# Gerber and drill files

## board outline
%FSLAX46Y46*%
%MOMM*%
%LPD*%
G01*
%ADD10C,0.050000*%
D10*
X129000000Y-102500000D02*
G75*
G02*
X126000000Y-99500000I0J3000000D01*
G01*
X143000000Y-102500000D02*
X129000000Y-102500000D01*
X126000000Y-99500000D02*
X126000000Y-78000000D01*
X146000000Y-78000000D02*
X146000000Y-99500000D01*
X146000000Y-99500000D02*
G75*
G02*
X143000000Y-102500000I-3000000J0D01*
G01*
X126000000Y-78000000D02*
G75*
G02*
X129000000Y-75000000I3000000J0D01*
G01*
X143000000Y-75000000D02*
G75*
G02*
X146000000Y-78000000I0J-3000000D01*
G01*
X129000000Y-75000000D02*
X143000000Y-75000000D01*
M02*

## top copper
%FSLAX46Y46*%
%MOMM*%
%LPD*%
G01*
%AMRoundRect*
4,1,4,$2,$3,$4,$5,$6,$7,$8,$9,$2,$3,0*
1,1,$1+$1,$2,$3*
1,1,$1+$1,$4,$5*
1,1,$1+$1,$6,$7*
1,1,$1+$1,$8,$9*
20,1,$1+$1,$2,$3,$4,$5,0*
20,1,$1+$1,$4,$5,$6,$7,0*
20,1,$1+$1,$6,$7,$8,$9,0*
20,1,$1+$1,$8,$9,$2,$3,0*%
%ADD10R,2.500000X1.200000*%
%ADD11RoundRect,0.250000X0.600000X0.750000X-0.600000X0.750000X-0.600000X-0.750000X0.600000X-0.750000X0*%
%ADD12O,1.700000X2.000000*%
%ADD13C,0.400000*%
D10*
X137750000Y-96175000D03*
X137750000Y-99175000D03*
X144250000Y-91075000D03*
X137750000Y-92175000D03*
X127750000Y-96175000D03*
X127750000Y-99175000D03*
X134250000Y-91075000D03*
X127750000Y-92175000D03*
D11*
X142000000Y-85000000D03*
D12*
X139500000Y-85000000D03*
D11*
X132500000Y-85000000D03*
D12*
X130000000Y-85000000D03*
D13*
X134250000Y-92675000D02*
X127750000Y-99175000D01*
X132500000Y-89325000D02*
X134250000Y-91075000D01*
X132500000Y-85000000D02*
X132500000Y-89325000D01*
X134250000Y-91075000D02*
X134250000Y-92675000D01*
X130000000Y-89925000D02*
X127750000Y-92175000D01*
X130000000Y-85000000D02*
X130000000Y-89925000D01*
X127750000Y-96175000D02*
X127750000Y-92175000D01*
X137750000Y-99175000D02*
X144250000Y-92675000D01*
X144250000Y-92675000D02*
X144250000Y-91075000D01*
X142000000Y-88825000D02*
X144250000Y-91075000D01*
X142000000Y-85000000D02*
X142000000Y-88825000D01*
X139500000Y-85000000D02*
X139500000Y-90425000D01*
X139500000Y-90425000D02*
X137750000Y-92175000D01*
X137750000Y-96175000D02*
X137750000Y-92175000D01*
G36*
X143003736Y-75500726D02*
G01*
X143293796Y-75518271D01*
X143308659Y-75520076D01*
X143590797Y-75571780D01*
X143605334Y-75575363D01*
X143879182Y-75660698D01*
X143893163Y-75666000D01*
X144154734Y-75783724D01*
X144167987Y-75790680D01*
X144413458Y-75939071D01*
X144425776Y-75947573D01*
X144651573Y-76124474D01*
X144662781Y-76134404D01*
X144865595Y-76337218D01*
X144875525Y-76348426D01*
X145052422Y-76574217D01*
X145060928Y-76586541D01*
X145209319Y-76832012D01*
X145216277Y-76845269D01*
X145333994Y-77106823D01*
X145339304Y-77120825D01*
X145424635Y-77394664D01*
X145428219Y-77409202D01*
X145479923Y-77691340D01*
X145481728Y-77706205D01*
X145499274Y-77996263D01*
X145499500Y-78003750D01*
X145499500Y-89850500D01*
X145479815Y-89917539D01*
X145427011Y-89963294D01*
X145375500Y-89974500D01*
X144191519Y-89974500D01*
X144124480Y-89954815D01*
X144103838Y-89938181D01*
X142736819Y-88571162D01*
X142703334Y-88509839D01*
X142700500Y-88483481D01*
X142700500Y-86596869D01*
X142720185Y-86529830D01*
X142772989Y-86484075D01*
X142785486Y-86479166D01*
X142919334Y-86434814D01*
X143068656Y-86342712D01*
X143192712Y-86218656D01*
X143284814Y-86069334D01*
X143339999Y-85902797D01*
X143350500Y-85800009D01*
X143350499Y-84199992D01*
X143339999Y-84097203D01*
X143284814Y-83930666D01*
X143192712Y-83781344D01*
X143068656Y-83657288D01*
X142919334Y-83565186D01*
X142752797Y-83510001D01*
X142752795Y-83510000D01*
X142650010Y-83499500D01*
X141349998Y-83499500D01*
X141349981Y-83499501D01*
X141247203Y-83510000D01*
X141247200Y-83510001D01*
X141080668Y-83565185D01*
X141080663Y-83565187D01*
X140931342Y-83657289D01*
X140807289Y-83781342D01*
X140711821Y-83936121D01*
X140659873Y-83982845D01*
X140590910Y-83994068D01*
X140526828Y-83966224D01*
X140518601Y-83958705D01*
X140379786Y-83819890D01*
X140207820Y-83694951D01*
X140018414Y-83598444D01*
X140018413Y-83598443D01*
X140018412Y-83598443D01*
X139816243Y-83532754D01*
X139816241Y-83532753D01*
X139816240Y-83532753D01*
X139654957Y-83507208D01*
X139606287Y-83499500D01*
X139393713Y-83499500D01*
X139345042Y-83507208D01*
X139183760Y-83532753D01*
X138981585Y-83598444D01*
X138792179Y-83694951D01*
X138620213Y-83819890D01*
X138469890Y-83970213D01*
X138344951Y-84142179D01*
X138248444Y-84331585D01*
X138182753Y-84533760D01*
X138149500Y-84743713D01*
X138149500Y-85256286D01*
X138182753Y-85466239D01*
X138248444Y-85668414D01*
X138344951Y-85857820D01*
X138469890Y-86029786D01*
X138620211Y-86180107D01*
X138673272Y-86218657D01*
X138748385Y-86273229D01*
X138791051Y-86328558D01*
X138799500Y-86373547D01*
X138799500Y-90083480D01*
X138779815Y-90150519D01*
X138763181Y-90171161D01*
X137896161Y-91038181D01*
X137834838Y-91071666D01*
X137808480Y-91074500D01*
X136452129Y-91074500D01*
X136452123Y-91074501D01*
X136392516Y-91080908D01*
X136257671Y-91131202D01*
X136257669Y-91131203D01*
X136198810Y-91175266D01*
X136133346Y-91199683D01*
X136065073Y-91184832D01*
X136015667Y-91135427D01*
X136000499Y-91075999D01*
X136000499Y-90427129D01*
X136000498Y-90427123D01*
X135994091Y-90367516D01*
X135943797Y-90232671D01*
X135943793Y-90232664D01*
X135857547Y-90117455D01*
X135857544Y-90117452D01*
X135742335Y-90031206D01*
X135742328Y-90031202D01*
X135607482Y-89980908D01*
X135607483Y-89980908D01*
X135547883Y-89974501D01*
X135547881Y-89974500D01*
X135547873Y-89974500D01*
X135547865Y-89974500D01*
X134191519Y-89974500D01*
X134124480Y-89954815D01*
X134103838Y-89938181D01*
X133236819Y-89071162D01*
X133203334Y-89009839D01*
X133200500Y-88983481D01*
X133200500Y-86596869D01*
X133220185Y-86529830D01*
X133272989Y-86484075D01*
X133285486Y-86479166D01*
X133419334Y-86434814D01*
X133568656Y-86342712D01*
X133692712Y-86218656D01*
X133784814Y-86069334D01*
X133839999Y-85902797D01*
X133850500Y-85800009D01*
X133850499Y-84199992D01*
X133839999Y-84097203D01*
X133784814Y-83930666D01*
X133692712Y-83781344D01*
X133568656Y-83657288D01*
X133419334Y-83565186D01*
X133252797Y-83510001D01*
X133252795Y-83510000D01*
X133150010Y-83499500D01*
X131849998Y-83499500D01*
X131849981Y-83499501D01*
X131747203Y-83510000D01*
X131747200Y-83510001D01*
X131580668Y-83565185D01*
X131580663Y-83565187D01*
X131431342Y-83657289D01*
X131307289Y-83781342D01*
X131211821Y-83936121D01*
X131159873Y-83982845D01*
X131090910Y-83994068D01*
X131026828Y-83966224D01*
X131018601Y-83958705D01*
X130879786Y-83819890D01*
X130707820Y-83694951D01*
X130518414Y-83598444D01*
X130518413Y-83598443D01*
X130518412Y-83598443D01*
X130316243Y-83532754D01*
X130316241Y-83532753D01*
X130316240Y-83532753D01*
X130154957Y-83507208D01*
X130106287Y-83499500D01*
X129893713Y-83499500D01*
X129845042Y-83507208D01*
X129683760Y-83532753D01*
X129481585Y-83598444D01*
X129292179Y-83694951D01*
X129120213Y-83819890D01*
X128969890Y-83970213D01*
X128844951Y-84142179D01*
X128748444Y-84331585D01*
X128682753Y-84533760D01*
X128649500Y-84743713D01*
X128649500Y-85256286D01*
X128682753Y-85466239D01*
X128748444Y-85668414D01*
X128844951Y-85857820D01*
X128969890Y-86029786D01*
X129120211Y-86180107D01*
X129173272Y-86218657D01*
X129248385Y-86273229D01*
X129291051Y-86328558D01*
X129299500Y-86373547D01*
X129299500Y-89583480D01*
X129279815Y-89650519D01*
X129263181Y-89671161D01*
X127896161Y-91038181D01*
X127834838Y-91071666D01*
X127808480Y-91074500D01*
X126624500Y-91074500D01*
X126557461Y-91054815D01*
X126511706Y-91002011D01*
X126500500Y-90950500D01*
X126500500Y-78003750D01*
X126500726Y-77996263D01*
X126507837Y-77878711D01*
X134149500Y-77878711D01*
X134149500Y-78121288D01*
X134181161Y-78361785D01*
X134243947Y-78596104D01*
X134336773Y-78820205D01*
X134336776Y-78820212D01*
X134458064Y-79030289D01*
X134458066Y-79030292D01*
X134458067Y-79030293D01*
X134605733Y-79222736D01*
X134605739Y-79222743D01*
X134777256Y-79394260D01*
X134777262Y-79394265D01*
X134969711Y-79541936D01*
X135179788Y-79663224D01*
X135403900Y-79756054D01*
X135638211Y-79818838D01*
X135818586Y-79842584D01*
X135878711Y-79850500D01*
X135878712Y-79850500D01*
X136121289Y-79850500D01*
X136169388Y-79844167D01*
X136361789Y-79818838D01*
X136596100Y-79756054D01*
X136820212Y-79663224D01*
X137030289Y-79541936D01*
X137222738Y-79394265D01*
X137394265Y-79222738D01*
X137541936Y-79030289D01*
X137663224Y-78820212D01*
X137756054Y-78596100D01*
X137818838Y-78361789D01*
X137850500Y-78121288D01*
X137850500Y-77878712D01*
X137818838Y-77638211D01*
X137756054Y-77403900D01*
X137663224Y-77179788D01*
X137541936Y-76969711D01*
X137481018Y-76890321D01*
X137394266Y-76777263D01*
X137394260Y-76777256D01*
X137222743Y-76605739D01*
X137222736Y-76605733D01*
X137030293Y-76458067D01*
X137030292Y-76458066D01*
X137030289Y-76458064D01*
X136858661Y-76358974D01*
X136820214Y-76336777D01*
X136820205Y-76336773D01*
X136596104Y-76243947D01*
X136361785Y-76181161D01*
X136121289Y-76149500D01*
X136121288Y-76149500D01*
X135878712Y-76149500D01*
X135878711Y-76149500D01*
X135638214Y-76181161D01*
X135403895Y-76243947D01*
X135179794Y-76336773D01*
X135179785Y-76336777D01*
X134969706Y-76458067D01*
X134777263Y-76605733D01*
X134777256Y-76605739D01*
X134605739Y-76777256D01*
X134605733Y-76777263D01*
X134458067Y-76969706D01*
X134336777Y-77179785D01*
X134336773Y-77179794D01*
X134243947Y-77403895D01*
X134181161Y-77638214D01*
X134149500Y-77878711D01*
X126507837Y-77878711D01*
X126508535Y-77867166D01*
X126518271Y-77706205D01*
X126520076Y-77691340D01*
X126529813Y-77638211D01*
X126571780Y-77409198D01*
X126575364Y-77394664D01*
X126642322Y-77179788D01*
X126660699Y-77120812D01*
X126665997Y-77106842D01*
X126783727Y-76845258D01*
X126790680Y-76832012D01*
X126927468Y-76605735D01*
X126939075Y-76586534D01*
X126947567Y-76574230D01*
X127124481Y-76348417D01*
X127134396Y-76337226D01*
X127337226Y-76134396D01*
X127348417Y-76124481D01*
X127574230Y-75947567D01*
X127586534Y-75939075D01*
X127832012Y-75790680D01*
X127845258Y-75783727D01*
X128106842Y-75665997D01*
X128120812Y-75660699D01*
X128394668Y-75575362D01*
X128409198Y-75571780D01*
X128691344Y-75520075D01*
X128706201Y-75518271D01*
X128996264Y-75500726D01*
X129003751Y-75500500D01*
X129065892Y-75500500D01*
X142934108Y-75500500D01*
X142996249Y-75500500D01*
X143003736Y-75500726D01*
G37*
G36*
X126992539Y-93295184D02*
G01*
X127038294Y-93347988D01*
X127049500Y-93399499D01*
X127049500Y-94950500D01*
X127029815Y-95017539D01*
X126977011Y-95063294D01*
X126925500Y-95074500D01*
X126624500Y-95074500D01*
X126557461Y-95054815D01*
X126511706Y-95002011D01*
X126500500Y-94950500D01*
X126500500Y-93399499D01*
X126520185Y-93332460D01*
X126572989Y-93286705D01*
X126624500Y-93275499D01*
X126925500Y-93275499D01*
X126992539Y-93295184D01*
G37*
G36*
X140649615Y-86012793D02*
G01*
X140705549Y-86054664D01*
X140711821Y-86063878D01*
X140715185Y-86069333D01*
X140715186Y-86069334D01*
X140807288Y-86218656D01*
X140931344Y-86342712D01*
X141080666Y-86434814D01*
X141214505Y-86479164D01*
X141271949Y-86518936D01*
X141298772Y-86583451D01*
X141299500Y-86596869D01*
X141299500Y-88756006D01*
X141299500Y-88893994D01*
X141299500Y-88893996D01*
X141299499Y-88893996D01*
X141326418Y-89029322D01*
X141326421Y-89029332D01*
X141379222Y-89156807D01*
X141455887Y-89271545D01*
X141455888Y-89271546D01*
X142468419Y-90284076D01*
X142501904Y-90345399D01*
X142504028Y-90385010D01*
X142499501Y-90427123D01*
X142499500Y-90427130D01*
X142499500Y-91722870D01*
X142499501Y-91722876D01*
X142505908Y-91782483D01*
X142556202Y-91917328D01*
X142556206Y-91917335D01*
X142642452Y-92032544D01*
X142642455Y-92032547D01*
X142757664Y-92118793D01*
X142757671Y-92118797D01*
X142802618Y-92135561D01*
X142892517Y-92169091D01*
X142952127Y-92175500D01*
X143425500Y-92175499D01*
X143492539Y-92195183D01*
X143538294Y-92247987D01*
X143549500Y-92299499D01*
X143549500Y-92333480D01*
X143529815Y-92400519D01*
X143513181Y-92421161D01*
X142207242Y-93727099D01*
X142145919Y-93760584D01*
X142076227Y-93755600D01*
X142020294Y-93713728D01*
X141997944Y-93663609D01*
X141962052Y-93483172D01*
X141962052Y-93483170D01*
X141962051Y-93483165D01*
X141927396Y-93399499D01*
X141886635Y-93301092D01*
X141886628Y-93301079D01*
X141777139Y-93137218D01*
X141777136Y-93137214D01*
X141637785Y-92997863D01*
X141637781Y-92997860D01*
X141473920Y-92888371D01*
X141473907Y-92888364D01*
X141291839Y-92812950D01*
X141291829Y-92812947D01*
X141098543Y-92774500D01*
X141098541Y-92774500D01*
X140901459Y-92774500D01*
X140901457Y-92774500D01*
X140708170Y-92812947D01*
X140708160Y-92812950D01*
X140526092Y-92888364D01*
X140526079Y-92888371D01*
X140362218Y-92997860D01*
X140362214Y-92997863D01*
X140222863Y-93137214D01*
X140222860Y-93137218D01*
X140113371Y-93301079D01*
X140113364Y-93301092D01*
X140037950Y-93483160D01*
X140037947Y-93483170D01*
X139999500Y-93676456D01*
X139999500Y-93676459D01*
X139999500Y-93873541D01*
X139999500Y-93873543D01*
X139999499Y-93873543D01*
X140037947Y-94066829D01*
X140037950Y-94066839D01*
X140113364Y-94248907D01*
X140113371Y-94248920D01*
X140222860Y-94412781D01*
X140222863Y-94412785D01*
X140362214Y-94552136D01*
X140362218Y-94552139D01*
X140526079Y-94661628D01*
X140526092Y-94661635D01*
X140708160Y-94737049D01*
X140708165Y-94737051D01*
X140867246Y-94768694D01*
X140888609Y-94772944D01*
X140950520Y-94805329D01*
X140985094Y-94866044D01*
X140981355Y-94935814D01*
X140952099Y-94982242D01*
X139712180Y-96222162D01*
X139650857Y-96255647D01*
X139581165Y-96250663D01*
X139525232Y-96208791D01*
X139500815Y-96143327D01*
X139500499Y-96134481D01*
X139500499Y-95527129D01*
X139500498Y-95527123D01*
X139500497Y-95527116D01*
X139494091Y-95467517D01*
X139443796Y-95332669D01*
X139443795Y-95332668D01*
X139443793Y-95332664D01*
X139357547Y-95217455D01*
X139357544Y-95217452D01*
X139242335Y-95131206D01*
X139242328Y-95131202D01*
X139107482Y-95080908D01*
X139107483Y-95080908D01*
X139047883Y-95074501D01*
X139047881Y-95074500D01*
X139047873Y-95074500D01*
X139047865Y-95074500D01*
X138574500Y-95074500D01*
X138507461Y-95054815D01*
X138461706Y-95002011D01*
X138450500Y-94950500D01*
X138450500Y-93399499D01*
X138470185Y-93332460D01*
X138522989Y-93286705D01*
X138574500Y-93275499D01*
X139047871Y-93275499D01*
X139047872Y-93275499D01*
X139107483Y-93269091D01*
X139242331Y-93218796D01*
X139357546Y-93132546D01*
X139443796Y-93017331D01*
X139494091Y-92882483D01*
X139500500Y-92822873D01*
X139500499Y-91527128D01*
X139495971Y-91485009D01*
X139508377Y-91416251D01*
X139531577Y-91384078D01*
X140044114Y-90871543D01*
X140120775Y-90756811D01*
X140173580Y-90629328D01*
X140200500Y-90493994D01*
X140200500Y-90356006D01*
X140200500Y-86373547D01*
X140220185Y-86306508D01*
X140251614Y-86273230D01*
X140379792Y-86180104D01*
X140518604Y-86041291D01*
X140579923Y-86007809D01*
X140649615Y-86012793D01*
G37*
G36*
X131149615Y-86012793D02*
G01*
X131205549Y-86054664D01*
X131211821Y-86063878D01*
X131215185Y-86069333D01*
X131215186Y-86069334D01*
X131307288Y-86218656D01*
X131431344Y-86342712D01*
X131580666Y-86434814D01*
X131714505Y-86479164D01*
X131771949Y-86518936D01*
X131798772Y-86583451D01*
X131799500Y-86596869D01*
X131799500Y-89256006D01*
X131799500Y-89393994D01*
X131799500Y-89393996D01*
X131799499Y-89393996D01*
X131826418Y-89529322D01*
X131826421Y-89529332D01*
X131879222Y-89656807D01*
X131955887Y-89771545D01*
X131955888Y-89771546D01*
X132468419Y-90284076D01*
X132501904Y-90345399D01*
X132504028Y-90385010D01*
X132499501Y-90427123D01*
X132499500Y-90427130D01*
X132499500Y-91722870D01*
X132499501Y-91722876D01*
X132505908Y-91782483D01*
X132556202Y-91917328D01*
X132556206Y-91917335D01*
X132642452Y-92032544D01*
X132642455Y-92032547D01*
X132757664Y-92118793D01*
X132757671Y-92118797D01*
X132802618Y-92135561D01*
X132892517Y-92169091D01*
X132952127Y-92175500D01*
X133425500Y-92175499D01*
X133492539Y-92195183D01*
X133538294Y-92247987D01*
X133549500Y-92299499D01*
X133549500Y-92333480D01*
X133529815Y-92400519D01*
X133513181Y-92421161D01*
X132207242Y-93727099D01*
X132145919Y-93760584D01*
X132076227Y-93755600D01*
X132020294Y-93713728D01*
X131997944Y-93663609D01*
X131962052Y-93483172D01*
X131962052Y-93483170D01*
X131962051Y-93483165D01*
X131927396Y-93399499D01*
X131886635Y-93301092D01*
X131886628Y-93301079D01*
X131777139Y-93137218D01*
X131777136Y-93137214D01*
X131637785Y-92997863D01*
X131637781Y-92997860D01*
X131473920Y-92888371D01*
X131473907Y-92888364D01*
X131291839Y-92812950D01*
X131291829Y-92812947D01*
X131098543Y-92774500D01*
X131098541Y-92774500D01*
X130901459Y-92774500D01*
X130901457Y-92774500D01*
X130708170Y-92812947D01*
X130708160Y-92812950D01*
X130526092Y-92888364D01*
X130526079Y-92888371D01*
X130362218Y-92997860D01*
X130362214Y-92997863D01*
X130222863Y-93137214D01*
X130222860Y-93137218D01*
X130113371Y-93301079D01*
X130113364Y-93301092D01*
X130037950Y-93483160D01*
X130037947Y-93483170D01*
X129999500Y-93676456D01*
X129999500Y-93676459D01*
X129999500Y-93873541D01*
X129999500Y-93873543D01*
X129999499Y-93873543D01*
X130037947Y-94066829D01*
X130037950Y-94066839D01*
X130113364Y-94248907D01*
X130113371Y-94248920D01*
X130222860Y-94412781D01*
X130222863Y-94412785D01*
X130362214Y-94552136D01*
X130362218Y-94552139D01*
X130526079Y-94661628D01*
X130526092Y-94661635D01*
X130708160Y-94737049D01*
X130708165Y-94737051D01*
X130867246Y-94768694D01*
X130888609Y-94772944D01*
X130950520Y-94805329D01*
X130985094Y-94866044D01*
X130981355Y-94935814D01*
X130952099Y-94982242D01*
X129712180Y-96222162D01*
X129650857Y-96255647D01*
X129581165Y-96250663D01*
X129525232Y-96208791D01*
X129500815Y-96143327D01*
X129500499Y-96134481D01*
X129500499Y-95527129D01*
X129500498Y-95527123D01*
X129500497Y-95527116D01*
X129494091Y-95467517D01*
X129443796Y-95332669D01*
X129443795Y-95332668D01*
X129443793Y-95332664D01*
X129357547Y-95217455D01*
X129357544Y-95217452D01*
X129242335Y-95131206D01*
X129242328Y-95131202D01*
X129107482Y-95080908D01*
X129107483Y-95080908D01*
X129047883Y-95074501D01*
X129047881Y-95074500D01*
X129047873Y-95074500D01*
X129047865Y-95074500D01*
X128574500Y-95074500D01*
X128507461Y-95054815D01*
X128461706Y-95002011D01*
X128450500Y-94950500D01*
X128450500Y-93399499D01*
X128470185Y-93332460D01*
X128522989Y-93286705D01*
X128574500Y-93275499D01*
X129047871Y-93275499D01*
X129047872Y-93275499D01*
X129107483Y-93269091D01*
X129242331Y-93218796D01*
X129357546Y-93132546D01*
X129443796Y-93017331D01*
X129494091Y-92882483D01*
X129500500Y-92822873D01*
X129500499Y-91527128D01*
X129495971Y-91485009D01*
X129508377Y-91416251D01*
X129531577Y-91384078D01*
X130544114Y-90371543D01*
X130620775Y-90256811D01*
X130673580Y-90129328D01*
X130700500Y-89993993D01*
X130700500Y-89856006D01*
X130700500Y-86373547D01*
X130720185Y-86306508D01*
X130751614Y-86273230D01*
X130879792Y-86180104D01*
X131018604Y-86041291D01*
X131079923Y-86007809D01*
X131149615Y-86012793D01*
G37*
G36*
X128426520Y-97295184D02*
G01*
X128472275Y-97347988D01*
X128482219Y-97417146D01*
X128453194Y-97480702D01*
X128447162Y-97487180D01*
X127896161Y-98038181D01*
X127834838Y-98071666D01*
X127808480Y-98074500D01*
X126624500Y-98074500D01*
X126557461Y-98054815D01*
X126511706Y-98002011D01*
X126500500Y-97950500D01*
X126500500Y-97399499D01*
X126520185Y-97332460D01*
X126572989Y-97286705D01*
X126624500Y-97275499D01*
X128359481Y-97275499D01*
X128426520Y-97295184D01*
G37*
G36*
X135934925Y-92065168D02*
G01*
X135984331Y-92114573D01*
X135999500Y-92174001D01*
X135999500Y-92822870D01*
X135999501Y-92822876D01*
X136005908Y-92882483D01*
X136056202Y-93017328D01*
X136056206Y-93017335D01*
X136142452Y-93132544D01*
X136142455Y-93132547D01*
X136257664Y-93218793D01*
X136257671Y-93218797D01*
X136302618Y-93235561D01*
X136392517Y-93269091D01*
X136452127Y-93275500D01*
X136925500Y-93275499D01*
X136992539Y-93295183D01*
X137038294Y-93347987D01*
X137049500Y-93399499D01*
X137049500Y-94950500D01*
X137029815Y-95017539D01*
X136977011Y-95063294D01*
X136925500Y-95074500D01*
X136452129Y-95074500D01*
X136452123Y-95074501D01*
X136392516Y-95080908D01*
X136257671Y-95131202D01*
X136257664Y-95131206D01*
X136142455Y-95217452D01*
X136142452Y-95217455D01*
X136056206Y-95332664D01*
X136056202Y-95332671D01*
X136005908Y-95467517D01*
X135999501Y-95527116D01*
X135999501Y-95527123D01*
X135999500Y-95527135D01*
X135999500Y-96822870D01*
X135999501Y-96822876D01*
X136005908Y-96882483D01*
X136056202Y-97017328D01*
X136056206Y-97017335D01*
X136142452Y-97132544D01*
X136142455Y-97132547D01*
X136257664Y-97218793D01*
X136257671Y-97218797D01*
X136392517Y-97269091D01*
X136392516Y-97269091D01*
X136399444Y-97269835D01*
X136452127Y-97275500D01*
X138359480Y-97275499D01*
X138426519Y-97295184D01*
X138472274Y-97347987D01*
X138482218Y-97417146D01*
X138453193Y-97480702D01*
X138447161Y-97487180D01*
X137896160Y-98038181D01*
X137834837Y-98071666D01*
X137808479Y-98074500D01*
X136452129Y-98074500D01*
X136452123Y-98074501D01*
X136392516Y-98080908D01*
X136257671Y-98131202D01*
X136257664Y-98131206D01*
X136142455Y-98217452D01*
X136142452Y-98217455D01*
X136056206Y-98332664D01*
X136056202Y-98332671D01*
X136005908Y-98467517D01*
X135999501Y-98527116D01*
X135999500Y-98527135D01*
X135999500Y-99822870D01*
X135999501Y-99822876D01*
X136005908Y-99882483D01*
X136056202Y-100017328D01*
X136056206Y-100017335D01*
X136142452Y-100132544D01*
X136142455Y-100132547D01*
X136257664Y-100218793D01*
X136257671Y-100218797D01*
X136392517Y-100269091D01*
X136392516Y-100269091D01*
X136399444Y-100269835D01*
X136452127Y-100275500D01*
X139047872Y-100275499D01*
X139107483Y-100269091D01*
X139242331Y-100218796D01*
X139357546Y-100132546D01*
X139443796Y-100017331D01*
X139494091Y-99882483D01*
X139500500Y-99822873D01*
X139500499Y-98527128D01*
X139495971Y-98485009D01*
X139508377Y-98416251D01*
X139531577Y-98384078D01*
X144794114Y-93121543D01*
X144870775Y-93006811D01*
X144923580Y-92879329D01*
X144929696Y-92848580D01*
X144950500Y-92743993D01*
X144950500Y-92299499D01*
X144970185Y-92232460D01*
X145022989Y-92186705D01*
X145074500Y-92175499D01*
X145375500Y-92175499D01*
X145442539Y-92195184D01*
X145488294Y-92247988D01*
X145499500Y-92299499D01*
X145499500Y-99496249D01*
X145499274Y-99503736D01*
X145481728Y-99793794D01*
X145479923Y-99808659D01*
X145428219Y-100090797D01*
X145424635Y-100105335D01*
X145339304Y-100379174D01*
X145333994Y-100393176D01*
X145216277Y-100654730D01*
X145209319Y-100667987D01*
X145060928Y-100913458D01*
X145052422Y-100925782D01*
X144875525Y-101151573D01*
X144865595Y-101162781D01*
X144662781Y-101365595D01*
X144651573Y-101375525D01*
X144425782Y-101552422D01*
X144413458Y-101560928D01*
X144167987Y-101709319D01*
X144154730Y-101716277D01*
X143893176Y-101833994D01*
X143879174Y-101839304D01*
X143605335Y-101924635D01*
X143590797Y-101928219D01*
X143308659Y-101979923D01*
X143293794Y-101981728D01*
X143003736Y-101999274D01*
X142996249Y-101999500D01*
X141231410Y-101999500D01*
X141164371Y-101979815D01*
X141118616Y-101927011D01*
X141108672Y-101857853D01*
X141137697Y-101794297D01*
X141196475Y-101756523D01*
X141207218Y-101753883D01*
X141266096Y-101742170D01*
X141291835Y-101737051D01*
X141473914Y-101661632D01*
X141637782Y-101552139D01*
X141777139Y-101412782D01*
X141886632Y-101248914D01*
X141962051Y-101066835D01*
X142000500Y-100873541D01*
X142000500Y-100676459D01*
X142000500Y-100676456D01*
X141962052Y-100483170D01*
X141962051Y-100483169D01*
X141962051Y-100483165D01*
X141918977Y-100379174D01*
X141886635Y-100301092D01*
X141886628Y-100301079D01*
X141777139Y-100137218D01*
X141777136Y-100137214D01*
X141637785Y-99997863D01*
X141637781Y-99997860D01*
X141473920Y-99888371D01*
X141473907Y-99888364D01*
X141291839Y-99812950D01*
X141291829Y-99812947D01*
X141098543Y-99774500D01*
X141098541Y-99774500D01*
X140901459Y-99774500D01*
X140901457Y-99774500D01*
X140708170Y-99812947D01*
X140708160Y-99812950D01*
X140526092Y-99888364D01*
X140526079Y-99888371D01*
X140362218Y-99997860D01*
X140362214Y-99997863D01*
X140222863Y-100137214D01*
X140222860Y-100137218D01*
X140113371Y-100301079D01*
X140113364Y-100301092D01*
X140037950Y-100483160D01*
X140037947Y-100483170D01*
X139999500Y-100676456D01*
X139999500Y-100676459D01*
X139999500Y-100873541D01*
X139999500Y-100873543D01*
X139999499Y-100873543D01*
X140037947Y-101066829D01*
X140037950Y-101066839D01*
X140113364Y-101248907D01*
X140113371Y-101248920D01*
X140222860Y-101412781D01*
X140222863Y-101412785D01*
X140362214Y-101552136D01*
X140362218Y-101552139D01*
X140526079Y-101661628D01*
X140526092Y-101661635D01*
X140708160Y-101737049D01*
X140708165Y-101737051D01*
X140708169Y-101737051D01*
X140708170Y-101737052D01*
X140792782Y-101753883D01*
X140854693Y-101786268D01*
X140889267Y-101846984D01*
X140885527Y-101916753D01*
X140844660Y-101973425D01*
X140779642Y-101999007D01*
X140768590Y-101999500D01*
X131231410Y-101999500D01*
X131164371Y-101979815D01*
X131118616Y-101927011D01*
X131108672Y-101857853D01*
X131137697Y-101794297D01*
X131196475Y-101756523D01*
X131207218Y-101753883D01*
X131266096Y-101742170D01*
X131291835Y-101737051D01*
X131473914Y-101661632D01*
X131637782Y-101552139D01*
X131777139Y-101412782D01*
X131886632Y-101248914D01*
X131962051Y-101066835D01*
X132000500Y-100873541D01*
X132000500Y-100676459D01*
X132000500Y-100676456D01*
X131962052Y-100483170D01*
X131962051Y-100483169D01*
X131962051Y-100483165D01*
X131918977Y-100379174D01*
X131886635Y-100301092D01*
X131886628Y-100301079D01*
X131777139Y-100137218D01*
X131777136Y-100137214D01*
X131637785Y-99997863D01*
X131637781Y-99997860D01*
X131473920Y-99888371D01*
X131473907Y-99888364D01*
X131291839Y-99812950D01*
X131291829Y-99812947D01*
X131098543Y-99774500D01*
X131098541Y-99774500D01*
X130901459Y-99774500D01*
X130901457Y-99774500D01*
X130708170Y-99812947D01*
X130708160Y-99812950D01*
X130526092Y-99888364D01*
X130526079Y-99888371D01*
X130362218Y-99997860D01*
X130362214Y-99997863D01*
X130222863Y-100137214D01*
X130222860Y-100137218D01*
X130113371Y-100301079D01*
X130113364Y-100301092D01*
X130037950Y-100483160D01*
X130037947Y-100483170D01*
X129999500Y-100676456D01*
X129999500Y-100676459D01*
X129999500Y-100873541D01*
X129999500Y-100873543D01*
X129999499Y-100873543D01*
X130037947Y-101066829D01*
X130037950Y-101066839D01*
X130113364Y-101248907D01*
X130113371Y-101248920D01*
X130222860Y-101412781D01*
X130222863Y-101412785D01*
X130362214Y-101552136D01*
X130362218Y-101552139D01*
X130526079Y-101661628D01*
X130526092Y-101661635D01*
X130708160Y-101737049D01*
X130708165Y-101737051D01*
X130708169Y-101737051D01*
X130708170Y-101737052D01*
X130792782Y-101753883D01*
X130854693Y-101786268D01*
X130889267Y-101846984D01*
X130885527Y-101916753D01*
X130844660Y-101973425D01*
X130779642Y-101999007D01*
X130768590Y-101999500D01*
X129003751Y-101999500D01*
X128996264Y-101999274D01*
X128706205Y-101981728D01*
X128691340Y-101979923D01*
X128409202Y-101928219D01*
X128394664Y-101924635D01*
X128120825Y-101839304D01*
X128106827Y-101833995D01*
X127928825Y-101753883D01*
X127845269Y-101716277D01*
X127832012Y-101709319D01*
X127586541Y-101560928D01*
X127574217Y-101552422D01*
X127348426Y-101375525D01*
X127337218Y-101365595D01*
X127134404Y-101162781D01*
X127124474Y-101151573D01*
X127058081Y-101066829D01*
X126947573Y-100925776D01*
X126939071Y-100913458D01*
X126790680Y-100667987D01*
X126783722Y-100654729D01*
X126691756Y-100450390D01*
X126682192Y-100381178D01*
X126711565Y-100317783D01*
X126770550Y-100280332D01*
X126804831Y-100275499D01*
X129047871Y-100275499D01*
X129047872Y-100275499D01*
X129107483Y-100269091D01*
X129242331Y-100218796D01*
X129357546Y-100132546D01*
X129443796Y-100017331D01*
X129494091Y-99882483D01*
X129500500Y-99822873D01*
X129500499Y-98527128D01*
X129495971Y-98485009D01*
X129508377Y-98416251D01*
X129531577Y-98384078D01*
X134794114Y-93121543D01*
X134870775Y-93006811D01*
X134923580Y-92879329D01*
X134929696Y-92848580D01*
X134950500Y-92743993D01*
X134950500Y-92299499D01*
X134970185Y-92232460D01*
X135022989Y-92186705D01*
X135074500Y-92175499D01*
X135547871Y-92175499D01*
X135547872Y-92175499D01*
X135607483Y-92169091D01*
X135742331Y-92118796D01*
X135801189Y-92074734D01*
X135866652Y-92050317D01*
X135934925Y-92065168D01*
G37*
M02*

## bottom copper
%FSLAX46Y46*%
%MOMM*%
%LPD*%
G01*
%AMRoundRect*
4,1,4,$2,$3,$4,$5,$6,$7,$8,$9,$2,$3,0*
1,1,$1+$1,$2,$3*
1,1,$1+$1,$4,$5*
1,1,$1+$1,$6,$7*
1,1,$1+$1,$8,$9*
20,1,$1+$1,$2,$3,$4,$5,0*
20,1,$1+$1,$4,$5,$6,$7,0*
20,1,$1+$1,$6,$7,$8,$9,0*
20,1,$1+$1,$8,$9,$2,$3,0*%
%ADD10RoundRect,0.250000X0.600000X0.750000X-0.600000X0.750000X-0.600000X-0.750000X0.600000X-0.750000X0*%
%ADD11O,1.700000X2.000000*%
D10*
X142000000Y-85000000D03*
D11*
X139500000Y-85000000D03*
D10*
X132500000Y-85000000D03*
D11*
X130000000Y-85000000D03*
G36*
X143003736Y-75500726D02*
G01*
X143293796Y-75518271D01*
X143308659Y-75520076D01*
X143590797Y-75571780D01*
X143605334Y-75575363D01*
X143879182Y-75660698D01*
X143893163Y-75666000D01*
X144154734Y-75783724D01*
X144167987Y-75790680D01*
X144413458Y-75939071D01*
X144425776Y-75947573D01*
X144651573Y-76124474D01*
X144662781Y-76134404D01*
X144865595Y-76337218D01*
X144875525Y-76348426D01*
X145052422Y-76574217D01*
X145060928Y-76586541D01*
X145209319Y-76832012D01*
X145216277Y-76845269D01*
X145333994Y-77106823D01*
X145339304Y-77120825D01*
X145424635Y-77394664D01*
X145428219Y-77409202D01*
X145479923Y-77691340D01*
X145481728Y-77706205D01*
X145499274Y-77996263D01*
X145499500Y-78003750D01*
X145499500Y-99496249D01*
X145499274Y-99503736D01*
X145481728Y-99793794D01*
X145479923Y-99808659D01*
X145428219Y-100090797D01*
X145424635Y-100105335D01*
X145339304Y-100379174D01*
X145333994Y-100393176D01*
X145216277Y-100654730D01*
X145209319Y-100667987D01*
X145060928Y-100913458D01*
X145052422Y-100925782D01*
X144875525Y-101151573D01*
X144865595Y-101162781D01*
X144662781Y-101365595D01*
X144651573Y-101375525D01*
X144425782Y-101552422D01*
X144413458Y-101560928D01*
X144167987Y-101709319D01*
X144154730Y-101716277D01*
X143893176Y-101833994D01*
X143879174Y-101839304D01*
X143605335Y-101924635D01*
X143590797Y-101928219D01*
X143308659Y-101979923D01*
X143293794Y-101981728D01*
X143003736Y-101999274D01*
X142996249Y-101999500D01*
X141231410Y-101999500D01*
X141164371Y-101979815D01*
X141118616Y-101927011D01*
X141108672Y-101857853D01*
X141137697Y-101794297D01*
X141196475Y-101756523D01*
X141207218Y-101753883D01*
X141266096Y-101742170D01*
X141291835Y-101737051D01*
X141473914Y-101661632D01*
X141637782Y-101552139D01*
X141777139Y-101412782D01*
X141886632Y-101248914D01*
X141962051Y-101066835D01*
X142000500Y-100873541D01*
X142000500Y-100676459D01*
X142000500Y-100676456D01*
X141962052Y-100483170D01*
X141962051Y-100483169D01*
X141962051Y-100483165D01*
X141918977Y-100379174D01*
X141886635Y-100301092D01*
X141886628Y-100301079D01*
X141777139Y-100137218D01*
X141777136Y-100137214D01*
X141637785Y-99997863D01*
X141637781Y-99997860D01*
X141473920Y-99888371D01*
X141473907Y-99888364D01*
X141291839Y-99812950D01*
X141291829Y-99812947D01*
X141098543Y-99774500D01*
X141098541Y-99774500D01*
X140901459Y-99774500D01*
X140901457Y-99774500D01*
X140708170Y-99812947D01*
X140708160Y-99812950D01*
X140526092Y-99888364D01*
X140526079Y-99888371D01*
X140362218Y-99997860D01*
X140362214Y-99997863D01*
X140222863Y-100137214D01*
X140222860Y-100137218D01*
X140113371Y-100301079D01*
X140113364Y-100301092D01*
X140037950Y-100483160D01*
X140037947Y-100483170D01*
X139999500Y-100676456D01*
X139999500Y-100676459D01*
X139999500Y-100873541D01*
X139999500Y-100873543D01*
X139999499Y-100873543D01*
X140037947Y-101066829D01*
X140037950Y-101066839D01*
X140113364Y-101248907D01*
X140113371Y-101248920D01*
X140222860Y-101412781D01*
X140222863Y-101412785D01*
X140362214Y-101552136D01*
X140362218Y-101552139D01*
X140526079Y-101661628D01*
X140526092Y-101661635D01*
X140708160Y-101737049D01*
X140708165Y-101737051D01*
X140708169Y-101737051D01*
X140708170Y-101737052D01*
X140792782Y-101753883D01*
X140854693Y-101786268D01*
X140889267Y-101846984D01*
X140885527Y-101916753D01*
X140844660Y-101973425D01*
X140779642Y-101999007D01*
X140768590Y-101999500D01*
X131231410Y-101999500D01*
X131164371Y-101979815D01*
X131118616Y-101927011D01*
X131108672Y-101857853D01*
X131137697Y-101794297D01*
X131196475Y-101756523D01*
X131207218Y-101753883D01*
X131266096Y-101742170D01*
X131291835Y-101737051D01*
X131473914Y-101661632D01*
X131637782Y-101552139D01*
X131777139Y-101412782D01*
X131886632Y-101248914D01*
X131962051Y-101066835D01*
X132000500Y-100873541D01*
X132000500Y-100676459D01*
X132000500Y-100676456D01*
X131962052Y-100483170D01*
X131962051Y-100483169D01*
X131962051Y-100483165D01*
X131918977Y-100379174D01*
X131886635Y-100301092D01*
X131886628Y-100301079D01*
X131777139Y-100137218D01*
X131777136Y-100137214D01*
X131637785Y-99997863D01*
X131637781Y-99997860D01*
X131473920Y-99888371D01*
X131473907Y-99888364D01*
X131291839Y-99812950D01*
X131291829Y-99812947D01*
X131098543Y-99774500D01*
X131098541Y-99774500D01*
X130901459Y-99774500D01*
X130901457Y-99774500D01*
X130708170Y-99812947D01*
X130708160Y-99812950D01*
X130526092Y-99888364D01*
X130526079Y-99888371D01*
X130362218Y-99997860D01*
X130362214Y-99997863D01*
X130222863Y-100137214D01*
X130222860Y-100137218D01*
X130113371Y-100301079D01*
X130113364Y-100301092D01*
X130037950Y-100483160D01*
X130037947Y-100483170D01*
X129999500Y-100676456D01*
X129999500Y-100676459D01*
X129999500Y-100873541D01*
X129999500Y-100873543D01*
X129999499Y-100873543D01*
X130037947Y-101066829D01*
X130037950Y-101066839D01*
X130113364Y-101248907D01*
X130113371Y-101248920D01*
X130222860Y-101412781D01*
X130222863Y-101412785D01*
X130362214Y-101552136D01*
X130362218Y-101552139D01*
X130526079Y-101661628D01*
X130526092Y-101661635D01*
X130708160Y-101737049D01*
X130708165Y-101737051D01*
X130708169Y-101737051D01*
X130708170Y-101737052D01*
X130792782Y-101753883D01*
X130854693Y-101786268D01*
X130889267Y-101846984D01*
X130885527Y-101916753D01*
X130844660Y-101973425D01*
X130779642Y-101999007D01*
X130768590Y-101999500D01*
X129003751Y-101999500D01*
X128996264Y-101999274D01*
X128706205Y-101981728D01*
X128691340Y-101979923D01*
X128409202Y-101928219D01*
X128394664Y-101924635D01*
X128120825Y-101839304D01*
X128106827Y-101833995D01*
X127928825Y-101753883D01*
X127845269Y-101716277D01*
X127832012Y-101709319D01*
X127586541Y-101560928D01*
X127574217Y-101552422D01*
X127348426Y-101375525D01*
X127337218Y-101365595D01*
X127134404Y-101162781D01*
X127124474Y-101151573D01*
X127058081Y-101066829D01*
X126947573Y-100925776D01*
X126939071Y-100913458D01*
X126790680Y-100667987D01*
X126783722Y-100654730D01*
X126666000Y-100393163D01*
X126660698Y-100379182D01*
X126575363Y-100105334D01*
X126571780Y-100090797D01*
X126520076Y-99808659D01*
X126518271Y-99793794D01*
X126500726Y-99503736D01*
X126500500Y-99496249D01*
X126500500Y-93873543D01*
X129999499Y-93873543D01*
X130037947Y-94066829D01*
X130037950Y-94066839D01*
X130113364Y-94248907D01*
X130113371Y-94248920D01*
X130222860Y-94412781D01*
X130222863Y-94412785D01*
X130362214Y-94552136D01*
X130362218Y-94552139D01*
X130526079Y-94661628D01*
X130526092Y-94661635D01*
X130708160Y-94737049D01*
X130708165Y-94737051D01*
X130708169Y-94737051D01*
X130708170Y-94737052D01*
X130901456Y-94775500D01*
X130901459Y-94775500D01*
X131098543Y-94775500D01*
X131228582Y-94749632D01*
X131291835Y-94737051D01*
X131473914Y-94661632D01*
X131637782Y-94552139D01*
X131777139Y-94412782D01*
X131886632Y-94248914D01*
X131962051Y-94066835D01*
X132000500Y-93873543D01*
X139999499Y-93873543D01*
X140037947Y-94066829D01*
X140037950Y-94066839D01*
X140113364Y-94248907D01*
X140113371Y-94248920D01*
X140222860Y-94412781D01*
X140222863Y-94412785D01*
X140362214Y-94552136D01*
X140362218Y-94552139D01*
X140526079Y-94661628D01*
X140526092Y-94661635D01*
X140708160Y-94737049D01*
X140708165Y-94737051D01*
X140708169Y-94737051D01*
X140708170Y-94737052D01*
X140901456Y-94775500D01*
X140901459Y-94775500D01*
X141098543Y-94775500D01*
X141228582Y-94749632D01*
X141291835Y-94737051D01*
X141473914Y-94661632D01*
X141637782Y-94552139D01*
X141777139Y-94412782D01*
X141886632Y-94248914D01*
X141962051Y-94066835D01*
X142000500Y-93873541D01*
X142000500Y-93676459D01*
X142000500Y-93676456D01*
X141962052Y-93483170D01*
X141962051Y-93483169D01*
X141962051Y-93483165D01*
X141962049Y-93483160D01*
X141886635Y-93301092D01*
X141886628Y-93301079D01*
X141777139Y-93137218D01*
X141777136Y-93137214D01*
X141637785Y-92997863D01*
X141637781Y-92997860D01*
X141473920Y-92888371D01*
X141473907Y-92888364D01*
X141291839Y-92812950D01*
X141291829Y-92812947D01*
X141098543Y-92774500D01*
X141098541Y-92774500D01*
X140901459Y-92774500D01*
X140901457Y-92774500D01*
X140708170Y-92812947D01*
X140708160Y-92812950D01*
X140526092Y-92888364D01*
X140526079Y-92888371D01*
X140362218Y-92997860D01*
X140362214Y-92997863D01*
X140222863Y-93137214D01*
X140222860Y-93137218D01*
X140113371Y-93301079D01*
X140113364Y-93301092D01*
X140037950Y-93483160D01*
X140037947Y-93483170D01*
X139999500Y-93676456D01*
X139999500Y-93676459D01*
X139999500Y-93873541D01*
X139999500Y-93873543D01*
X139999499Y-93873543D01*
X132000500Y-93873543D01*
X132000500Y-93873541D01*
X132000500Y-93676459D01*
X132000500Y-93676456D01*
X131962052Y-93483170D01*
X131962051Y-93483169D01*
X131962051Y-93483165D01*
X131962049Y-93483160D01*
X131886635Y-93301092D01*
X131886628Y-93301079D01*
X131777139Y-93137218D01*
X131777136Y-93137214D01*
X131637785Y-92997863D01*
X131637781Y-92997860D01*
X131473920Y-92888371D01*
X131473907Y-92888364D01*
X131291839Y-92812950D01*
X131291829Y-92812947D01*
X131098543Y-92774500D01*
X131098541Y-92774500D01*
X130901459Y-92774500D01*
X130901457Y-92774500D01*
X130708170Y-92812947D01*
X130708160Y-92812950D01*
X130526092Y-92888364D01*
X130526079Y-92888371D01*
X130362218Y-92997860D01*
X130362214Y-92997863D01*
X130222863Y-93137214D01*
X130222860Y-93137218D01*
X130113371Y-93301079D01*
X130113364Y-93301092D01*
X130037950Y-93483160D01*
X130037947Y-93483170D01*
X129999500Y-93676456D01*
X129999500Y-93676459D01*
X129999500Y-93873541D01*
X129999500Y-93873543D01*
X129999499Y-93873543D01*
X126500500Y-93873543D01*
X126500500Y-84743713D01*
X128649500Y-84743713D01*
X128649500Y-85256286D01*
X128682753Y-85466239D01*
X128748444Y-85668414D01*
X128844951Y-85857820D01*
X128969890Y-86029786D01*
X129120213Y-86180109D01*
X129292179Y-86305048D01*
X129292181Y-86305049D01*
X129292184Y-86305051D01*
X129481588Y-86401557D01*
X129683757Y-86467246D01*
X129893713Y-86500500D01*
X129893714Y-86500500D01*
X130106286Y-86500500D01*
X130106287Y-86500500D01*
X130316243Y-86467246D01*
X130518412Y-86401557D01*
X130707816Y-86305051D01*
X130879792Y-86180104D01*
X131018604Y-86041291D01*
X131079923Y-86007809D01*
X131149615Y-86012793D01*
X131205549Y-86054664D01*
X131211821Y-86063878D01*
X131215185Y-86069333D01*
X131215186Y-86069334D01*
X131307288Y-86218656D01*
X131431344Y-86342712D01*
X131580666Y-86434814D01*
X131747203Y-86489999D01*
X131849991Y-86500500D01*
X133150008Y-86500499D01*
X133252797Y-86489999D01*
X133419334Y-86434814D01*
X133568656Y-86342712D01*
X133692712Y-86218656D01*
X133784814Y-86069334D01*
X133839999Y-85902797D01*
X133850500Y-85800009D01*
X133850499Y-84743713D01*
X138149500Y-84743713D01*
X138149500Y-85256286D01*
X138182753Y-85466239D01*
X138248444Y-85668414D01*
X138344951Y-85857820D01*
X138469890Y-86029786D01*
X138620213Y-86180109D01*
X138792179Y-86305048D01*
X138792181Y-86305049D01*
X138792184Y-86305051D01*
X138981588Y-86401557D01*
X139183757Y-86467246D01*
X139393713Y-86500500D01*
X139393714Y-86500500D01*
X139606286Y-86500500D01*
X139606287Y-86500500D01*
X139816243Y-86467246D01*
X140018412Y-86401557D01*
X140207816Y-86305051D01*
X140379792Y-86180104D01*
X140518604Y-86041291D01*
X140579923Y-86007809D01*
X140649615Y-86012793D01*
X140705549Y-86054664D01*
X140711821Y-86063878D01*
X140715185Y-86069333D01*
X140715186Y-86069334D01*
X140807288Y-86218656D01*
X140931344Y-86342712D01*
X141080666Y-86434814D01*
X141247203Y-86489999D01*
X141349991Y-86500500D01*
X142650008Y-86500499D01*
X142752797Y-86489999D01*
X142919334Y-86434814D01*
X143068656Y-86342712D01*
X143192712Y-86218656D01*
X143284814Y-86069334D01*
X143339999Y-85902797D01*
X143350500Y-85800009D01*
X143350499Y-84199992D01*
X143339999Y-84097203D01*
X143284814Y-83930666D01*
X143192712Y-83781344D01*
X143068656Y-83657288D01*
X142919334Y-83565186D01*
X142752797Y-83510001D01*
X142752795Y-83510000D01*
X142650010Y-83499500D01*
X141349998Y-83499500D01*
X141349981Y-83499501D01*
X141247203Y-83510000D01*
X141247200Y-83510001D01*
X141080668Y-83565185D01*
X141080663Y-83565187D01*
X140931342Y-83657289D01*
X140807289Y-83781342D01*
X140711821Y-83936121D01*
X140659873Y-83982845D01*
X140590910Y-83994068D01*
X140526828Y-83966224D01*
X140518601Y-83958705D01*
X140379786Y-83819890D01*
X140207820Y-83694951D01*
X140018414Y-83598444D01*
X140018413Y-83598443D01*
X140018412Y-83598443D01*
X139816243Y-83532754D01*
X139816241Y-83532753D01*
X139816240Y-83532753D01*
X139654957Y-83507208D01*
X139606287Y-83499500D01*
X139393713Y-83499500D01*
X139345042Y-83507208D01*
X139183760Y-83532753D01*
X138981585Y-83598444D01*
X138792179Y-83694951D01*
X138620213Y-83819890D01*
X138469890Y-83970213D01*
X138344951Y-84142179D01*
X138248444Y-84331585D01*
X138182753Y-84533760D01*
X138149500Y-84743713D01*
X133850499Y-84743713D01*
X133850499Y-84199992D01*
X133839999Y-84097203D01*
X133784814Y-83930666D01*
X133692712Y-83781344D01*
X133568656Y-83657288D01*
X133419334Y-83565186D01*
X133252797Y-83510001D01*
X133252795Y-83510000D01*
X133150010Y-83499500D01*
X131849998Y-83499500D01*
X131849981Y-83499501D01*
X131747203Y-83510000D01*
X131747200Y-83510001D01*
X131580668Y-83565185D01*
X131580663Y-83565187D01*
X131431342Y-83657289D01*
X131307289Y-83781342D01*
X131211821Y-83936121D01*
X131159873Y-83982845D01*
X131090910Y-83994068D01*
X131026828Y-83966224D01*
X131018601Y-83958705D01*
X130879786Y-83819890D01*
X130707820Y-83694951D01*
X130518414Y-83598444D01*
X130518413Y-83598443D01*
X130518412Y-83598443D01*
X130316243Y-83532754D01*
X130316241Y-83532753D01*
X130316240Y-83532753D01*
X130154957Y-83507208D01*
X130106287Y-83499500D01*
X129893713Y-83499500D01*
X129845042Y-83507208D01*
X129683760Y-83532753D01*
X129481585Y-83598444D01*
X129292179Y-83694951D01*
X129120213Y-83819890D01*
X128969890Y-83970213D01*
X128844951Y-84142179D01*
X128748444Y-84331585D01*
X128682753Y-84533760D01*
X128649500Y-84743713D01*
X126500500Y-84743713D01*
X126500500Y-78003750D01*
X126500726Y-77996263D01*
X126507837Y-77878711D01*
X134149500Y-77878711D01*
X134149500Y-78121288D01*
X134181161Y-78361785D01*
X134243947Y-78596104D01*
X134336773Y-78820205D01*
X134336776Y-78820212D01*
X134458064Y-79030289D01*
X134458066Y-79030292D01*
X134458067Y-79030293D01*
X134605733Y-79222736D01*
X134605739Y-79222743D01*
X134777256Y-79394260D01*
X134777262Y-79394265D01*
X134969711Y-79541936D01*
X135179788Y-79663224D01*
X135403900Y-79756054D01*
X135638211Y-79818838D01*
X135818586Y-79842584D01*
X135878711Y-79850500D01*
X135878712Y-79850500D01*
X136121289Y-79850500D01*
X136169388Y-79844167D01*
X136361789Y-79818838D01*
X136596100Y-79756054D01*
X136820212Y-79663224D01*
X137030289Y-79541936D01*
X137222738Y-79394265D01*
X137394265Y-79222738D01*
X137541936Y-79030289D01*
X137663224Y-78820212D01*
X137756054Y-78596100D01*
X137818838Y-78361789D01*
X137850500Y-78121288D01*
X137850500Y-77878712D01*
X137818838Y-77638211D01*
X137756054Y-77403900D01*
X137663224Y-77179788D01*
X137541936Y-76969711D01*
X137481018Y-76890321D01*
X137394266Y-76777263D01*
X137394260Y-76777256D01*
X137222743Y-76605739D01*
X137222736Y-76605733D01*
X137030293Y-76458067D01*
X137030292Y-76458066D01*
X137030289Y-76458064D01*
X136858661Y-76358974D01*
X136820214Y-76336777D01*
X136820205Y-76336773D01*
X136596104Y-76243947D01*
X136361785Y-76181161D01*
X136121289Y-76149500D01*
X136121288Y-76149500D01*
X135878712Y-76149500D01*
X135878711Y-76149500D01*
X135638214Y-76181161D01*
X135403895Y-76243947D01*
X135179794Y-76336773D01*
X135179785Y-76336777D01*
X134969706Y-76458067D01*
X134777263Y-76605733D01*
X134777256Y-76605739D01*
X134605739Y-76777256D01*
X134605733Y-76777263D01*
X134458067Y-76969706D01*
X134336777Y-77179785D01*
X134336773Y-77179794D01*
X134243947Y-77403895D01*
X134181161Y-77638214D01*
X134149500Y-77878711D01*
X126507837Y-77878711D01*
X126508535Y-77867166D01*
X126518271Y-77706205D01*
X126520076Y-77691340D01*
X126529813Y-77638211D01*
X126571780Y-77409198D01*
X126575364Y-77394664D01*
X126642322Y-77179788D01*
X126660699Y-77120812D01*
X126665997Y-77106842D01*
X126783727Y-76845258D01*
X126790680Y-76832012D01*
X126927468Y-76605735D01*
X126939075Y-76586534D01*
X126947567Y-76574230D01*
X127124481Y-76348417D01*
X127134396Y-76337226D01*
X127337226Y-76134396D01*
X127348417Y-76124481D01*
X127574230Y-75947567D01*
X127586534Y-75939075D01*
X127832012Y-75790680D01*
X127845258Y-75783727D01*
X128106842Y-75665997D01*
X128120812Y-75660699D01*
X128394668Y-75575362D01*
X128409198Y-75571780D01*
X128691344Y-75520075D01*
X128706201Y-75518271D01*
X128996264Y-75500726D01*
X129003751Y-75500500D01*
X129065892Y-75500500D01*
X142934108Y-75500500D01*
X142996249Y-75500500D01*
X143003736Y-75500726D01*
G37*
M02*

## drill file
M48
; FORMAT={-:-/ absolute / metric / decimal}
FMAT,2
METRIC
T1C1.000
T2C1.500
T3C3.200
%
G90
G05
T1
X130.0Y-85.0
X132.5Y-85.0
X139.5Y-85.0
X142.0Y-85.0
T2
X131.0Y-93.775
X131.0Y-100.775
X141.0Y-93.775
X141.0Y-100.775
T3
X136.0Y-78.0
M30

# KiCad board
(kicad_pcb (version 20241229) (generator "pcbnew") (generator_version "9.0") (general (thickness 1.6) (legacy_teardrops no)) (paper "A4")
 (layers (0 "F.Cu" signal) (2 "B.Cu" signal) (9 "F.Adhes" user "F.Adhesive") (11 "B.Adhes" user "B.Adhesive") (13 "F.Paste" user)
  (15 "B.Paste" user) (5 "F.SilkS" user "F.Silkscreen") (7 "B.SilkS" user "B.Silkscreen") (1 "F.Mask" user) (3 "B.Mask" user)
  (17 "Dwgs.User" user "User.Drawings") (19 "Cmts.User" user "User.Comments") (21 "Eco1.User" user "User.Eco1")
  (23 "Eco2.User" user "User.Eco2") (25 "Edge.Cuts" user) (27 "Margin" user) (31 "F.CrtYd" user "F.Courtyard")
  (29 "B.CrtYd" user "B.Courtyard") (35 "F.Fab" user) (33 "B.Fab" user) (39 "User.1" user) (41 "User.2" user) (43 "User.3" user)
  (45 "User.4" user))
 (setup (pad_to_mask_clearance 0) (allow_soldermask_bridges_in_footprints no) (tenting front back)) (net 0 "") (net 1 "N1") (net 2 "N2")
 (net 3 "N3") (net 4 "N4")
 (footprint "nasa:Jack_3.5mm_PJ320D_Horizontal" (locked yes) (layer "F.Cu") (at 141 96 90)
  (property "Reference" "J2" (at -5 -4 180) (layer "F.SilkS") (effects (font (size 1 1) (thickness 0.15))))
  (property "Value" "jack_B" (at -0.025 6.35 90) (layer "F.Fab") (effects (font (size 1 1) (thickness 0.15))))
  (pad "" np_thru_hole circle (at -4.775 0 90) (size 1.5 1.5) (drill 1.5) (layers "*.Cu" "*.Mask"))
  (pad "" np_thru_hole circle (at 2.225 0 90) (size 1.5 1.5) (drill 1.5) (layers "*.Cu" "*.Mask"))
  (pad "R1" smd rect (at -0.175 -3.25 90) (size 1.2 2.5) (layers "F.Cu" "F.Mask" "F.Paste") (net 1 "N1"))
  (pad "R2" smd rect (at -3.175 -3.25 90) (size 1.2 2.5) (layers "F.Cu" "F.Mask" "F.Paste") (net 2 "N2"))
  (pad "S" smd rect (at 4.925 3.25 90) (size 1.2 2.5) (layers "F.Cu" "F.Mask" "F.Paste") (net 2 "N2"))
  (pad "T" smd rect (at 3.825 -3.25 90) (size 1.2 2.5) (layers "F.Cu" "F.Mask" "F.Paste") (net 1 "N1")))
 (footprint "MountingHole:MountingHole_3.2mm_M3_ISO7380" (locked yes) (layer "F.Cu") (at 136 78)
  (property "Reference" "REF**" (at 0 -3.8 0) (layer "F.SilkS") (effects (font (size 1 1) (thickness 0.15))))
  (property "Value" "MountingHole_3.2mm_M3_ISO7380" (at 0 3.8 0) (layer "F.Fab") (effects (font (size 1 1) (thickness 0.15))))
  (pad "" np_thru_hole circle (at 0 0) (size 3.2 3.2) (drill 3.2) (layers "*.Cu" "*.Mask")))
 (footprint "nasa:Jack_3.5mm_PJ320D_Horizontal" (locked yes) (layer "F.Cu") (at 131 96 90)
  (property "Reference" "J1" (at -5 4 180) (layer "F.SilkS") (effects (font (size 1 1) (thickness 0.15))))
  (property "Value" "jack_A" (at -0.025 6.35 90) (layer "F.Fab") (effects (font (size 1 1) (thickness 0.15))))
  (pad "" np_thru_hole circle (at -4.775 0 90) (size 1.5 1.5) (drill 1.5) (layers "*.Cu" "*.Mask"))
  (pad "" np_thru_hole circle (at 2.225 0 90) (size 1.5 1.5) (drill 1.5) (layers "*.Cu" "*.Mask"))
  (pad "R1" smd rect (at -0.175 -3.25 90) (size 1.2 2.5) (layers "F.Cu" "F.Mask" "F.Paste") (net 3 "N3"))
  (pad "R2" smd rect (at -3.175 -3.25 90) (size 1.2 2.5) (layers "F.Cu" "F.Mask" "F.Paste") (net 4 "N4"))
  (pad "S" smd rect (at 4.925 3.25 90) (size 1.2 2.5) (layers "F.Cu" "F.Mask" "F.Paste") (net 4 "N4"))
  (pad "T" smd rect (at 3.825 -3.25 90) (size 1.2 2.5) (layers "F.Cu" "F.Mask" "F.Paste") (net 3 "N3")))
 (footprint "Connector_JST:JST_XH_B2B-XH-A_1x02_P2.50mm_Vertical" (layer "B.Cu") (at 142 85 180)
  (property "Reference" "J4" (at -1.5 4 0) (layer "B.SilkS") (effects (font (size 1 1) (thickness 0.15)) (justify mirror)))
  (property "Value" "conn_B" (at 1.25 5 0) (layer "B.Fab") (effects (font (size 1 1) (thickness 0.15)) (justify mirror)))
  (pad "1" thru_hole roundrect (at 0 0 180) (size 1.7 2) (drill 1) (layers "*.Cu" "*.Mask") (remove_unused_layers no)
   (roundrect_rratio 0.147059) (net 2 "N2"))
  (pad "2" thru_hole oval (at 2.5 0 180) (size 1.7 2) (drill 1) (layers "*.Cu" "*.Mask") (remove_unused_layers no) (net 1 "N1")))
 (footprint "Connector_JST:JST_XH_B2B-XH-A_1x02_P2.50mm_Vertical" (layer "B.Cu") (at 132.5 85 180)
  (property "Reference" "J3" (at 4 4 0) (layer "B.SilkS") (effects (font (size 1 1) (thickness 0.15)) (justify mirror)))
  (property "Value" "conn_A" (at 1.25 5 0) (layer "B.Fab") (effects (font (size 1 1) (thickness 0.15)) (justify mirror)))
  (pad "1" thru_hole roundrect (at 0 0 180) (size 1.7 2) (drill 1) (layers "*.Cu" "*.Mask") (remove_unused_layers no)
   (roundrect_rratio 0.147059) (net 4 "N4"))
  (pad "2" thru_hole oval (at 2.5 0 180) (size 1.7 2) (drill 1) (layers "*.Cu" "*.Mask") (remove_unused_layers no) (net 3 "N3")))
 (gr_arc (start 129 102.5) (mid 126.87868 101.62132) (end 126 99.5) (stroke (width 0.05) (type default)) (layer "Edge.Cuts"))
 (gr_line (start 143 102.5) (end 129 102.5) (stroke (width 0.05) (type default)) (layer "Edge.Cuts"))
 (gr_line (start 126 99.5) (end 126 78) (stroke (width 0.05) (type default)) (layer "Edge.Cuts"))
 (gr_line (start 146 78) (end 146 99.5) (stroke (width 0.05) (type default)) (layer "Edge.Cuts"))
 (gr_arc (start 146 99.5) (mid 145.12132 101.62132) (end 143 102.5) (stroke (width 0.05) (type default)) (layer "Edge.Cuts"))
 (gr_arc (start 126 78) (mid 126.87868 75.87868) (end 129 75) (stroke (width 0.05) (type default)) (layer "Edge.Cuts"))
 (gr_arc (start 143 75) (mid 145.12132 75.87868) (end 146 78) (stroke (width 0.05) (type default)) (layer "Edge.Cuts"))
 (gr_line (start 129 75) (end 143 75) (stroke (width 0.05) (type default)) (layer "Edge.Cuts"))
 (segment (start 134.25 92.675) (end 127.75 99.175) (width 0.4) (layer "F.Cu") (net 4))
 (segment (start 132.5 89.325) (end 134.25 91.075) (width 0.4) (layer "F.Cu") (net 4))
 (segment (start 132.5 85) (end 132.5 89.325) (width 0.4) (layer "F.Cu") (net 4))
 (segment (start 134.25 91.075) (end 134.25 92.675) (width 0.4) (layer "F.Cu") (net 4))
 (segment (start 130 89.925) (end 127.75 92.175) (width 0.4) (layer "F.Cu") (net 3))
 (segment (start 130 85) (end 130 89.925) (width 0.4) (layer "F.Cu") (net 3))
 (segment (start 127.75 96.175) (end 127.75 92.175) (width 0.4) (layer "F.Cu") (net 3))
 (segment (start 137.75 99.175) (end 144.25 92.675) (width 0.4) (layer "F.Cu") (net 2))
 (segment (start 144.25 92.675) (end 144.25 91.075) (width 0.4) (layer "F.Cu") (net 2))
 (segment (start 142 88.825) (end 144.25 91.075) (width 0.4) (layer "F.Cu") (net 2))
 (segment (start 142 85) (end 142 88.825) (width 0.4) (layer "F.Cu") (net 2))
 (segment (start 139.5 85) (end 139.5 90.425) (width 0.4) (layer "F.Cu") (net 1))
 (segment (start 139.5 90.425) (end 137.75 92.175) (width 0.4) (layer "F.Cu") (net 1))
 (segment (start 137.75 96.175) (end 137.75 92.175) (width 0.4) (layer "F.Cu") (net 1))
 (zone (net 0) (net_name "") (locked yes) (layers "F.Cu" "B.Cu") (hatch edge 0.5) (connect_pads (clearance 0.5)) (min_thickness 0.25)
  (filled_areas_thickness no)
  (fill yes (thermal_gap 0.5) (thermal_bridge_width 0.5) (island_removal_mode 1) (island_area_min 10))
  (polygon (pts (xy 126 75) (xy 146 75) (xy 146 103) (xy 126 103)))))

